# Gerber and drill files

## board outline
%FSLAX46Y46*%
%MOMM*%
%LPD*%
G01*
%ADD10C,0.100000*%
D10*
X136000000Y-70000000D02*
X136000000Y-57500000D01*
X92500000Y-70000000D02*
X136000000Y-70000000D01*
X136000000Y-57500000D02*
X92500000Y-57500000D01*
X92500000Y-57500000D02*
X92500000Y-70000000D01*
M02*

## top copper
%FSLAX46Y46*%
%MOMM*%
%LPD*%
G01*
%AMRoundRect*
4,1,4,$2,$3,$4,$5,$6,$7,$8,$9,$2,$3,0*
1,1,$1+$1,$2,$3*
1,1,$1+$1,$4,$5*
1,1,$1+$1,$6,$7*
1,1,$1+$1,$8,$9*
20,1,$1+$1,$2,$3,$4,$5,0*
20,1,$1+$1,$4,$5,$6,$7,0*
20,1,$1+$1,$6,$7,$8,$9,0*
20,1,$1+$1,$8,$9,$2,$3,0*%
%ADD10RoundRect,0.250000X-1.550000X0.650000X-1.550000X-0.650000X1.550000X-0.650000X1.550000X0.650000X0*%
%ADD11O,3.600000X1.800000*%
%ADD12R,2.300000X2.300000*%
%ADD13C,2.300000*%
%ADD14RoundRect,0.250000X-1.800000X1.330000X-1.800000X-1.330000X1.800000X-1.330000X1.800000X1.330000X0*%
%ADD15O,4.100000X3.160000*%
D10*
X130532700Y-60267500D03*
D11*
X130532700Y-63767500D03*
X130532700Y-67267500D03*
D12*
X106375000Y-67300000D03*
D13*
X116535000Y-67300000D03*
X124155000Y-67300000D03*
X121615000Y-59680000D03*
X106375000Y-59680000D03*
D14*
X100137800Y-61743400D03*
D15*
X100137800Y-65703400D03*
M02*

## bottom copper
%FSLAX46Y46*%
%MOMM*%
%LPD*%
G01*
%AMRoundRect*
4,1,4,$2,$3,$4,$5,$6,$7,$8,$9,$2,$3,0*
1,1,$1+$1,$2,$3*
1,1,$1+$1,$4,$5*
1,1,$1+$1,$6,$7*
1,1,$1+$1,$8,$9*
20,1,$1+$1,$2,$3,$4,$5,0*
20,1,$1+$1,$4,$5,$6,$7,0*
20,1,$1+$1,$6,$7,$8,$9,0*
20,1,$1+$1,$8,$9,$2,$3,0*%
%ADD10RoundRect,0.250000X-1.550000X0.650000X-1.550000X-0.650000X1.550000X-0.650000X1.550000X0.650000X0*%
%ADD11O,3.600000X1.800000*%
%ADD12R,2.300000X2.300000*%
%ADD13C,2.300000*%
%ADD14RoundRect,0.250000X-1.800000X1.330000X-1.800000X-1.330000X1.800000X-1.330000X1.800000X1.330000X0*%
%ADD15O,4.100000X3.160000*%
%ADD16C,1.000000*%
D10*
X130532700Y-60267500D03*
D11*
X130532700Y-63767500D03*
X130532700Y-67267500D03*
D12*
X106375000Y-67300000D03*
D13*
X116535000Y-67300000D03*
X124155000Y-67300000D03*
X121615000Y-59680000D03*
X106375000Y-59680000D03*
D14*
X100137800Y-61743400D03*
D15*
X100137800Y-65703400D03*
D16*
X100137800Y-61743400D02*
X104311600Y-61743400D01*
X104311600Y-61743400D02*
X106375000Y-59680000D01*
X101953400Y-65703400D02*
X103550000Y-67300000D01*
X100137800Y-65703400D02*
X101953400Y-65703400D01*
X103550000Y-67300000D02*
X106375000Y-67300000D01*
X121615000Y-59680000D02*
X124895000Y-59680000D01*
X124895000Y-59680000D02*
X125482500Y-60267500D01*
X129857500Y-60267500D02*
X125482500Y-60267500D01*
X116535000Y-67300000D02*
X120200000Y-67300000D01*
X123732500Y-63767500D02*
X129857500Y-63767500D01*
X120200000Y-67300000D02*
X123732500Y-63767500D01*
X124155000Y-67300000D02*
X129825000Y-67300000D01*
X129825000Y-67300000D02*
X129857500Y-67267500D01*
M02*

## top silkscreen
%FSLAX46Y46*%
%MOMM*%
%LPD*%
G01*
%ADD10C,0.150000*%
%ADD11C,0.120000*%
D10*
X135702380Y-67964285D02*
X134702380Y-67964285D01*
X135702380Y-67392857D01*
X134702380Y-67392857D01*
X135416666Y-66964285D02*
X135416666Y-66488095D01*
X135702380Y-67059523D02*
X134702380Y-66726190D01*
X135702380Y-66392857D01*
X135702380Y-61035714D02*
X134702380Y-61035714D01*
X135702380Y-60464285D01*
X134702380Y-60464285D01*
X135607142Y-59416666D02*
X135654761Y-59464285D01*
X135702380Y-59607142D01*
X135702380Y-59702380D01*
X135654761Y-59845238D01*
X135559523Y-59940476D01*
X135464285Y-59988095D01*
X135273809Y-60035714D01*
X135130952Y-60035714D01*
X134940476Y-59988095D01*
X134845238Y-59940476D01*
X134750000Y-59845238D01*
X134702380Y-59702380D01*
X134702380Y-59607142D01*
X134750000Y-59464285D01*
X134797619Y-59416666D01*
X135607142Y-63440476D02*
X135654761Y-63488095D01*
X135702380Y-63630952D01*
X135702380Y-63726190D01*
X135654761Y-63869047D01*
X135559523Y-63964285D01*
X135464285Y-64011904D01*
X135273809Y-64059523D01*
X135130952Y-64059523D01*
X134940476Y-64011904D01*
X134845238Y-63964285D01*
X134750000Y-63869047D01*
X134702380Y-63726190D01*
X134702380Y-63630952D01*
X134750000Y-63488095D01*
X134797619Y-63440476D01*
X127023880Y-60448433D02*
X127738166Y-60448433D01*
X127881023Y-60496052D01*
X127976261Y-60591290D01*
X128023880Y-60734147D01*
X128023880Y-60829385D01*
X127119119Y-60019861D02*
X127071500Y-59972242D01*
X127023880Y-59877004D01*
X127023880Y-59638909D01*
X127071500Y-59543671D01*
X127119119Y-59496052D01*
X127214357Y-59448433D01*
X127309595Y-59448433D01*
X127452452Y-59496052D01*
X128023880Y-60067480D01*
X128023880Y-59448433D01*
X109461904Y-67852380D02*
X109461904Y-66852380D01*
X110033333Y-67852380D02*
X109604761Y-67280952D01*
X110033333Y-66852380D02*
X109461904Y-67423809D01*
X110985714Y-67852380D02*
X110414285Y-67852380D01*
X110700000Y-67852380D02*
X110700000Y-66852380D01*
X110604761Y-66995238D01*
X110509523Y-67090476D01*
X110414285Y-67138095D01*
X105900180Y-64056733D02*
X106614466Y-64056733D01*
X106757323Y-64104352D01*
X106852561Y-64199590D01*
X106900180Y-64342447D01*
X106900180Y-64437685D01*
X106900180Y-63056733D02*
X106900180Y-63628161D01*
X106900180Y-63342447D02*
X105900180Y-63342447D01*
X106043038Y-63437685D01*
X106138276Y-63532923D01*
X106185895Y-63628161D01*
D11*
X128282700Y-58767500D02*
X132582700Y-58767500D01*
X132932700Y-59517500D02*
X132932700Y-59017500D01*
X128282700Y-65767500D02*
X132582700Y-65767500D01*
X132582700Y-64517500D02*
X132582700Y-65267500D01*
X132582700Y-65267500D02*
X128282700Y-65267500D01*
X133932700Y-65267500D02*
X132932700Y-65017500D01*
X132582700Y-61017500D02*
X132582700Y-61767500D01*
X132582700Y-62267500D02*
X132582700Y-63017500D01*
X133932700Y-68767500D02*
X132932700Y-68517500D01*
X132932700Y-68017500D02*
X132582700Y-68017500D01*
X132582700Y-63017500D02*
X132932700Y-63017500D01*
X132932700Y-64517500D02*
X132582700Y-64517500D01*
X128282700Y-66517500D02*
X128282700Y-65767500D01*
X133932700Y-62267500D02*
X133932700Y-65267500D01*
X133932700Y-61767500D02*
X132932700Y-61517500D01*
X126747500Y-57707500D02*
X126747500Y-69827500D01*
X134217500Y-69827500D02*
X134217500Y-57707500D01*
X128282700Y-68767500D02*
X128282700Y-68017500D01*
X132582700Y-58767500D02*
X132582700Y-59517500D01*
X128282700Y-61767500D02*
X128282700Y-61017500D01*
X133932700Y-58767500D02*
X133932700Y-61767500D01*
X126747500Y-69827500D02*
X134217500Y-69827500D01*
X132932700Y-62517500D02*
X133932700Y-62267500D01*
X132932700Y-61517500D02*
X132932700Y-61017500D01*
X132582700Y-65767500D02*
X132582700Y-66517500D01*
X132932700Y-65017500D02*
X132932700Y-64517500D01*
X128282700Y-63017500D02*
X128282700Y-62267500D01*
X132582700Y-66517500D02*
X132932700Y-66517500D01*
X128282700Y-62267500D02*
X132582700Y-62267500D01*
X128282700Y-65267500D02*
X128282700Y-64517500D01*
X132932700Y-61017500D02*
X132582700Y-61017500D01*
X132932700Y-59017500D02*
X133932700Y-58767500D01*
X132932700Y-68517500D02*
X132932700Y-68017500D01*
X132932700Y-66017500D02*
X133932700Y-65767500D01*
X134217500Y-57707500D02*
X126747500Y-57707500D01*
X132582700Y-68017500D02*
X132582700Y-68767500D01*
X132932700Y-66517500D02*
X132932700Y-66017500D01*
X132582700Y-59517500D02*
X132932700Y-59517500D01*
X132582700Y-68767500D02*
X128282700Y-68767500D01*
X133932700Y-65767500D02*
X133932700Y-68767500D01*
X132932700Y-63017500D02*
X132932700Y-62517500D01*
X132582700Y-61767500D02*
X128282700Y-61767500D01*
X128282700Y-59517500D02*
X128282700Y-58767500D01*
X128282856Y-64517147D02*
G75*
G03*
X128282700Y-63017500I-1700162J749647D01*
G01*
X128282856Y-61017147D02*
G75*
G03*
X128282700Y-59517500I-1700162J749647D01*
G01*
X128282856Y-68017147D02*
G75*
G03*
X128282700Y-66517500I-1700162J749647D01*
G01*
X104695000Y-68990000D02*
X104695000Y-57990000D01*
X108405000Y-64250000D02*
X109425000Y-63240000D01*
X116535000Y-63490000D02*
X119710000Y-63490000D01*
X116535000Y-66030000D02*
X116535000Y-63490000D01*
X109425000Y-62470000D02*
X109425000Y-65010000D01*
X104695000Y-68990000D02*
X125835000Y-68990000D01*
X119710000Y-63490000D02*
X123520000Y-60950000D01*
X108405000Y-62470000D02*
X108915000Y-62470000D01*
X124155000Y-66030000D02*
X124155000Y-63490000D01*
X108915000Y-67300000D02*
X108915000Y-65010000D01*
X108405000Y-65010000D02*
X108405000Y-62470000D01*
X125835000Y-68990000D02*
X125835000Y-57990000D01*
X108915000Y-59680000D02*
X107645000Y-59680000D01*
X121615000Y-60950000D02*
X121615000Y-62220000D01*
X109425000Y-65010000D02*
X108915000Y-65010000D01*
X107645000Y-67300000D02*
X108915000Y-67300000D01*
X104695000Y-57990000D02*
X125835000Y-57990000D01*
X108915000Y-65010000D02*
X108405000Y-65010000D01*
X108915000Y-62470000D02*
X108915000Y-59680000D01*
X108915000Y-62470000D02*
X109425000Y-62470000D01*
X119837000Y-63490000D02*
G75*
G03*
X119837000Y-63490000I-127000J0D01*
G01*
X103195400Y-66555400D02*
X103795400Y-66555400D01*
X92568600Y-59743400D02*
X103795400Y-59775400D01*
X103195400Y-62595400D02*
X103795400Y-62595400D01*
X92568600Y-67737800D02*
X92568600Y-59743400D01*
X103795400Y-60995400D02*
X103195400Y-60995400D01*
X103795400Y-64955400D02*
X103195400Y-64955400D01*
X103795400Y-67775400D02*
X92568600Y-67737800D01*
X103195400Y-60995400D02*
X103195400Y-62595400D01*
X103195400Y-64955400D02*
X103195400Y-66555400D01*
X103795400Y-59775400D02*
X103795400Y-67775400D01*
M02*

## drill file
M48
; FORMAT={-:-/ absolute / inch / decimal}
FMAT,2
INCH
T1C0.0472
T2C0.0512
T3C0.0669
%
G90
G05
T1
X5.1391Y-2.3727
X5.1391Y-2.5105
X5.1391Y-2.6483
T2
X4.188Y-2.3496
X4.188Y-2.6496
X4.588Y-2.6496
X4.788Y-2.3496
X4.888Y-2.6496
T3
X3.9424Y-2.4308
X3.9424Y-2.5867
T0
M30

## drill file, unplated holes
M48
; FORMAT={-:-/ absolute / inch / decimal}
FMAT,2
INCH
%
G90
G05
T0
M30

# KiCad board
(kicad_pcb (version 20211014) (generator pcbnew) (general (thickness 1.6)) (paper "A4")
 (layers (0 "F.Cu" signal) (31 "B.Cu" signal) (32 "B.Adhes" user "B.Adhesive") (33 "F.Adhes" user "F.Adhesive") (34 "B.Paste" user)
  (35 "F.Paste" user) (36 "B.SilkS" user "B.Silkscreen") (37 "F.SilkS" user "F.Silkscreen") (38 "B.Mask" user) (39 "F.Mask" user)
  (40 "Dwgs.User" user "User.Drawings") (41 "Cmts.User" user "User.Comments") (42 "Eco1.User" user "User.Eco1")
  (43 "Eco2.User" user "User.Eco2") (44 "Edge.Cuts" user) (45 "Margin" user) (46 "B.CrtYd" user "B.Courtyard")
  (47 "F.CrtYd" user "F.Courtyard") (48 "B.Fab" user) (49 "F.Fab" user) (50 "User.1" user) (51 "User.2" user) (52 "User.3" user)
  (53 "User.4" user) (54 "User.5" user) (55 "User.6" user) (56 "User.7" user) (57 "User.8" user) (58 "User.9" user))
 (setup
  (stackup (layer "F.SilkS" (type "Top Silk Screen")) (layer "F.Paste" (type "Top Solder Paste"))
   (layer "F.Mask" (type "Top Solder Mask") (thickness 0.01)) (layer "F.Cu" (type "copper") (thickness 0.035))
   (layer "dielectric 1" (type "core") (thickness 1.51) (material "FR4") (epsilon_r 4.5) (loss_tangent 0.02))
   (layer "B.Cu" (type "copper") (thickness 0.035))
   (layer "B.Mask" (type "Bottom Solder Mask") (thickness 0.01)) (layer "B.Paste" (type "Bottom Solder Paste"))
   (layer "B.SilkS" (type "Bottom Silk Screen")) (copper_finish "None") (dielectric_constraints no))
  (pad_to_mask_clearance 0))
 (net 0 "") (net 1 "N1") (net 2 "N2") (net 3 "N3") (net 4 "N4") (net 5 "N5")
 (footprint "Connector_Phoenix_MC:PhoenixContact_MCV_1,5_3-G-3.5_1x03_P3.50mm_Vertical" (layer "F.Cu") (at 129.8575 60.2675 -90)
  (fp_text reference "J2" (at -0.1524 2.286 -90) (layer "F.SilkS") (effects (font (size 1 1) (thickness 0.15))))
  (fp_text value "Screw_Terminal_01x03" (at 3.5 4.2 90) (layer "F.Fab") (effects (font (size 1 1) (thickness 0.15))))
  (fp_line (start -1.5 1.5748) (end -1.5 -2.7252) (layer "F.SilkS") (width 0.12))
  (fp_line (start -0.75 -3.0752) (end -1.25 -3.0752) (layer "F.SilkS") (width 0.12))
  (fp_line (start 5.5 1.5748) (end 5.5 -2.7252) (layer "F.SilkS") (width 0.12))
  (fp_line (start 4.25 -2.7252) (end 5 -2.7252) (layer "F.SilkS") (width 0.12))
  (fp_line (start 5 -2.7252) (end 5 1.5748) (layer "F.SilkS") (width 0.12))
  (fp_line (start 5 -4.0752) (end 4.75 -3.0752) (layer "F.SilkS") (width 0.12))
  (fp_line (start 0.75 -2.7252) (end 1.5 -2.7252) (layer "F.SilkS") (width 0.12))
  (fp_line (start 2 -2.7252) (end 2.75 -2.7252) (layer "F.SilkS") (width 0.12))
  (fp_line (start 8.5 -4.0752) (end 8.25 -3.0752) (layer "F.SilkS") (width 0.12))
  (fp_line (start 7.75 -3.0752) (end 7.75 -2.7252) (layer "F.SilkS") (width 0.12))
  (fp_line (start 2.75 -2.7252) (end 2.75 -3.0752) (layer "F.SilkS") (width 0.12))
  (fp_line (start 4.25 -3.0752) (end 4.25 -2.7252) (layer "F.SilkS") (width 0.12))
  (fp_line (start 6.25 1.5748) (end 5.5 1.5748) (layer "F.SilkS") (width 0.12))
  (fp_line (start 2 -4.0752) (end 5 -4.0752) (layer "F.SilkS") (width 0.12))
  (fp_line (start 1.5 -4.0752) (end 1.25 -3.0752) (layer "F.SilkS") (width 0.12))
  (fp_line (start -2.56 3.11) (end 9.56 3.11) (layer "F.SilkS") (width 0.12))
  (fp_line (start 9.56 -4.36) (end -2.56 -4.36) (layer "F.SilkS") (width 0.12))
  (fp_line (start 8.5 1.5748) (end 7.75 1.5748) (layer "F.SilkS") (width 0.12))
  (fp_line (start -1.5 -2.7252) (end -0.75 -2.7252) (layer "F.SilkS") (width 0.12))
  (fp_line (start 1.5 1.5748) (end 0.75 1.5748) (layer "F.SilkS") (width 0.12))
  (fp_line (start -1.5 -4.0752) (end 1.5 -4.0752) (layer "F.SilkS") (width 0.12))
  (fp_line (start 9.56 3.11) (end 9.56 -4.36) (layer "F.SilkS") (width 0.12))
  (fp_line (start 2.25 -3.0752) (end 2 -4.0752) (layer "F.SilkS") (width 0.12))
  (fp_line (start 1.25 -3.0752) (end 0.75 -3.0752) (layer "F.SilkS") (width 0.12))
  (fp_line (start 5.5 -2.7252) (end 6.25 -2.7252) (layer "F.SilkS") (width 0.12))
  (fp_line (start 4.75 -3.0752) (end 4.25 -3.0752) (layer "F.SilkS") (width 0.12))
  (fp_line (start 2.75 1.5748) (end 2 1.5748) (layer "F.SilkS") (width 0.12))
  (fp_line (start 6.25 -2.7252) (end 6.25 -3.0752) (layer "F.SilkS") (width 0.12))
  (fp_line (start 2 1.5748) (end 2 -2.7252) (layer "F.SilkS") (width 0.12))
  (fp_line (start 5 1.5748) (end 4.25 1.5748) (layer "F.SilkS") (width 0.12))
  (fp_line (start 0.75 -3.0752) (end 0.75 -2.7252) (layer "F.SilkS") (width 0.12))
  (fp_line (start -1.25 -3.0752) (end -1.5 -4.0752) (layer "F.SilkS") (width 0.12))
  (fp_line (start 8.25 -3.0752) (end 7.75 -3.0752) (layer "F.SilkS") (width 0.12))
  (fp_line (start 5.75 -3.0752) (end 5.5 -4.0752) (layer "F.SilkS") (width 0.12))
  (fp_line (start -2.56 -4.36) (end -2.56 3.11) (layer "F.SilkS") (width 0.12))
  (fp_line (start 7.75 -2.7252) (end 8.5 -2.7252) (layer "F.SilkS") (width 0.12))
  (fp_line (start 6.25 -3.0752) (end 5.75 -3.0752) (layer "F.SilkS") (width 0.12))
  (fp_line (start -0.75 -2.7252) (end -0.75 -3.0752) (layer "F.SilkS") (width 0.12))
  (fp_line (start 8.5 -2.7252) (end 8.5 1.5748) (layer "F.SilkS") (width 0.12))
  (fp_line (start 5.5 -4.0752) (end 8.5 -4.0752) (layer "F.SilkS") (width 0.12))
  (fp_line (start 2.75 -3.0752) (end 2.25 -3.0752) (layer "F.SilkS") (width 0.12))
  (fp_line (start 1.5 -2.7252) (end 1.5 1.5748) (layer "F.SilkS") (width 0.12))
  (fp_line (start -0.75 1.5748) (end -1.5 1.5748) (layer "F.SilkS") (width 0.12))
  (fp_arc (start 2.75 1.5748) (mid 3.499807 1.41671) (end 4.249647 1.574644) (layer "F.SilkS") (width 0.12))
  (fp_arc (start -0.75 1.5748) (mid -0.000193 1.41671) (end 0.749647 1.574644) (layer "F.SilkS") (width 0.12))
  (fp_arc (start 6.25 1.5748) (mid 6.999807 1.41671) (end 7.749647 1.574644) (layer "F.SilkS") (width 0.12))
  (pad "1" thru_hole roundrect (at 0 -0.6752 270) (size 1.8 3.6) (drill 1.2) (layers *.Cu *.Mask) (roundrect_rratio 0.1388888889)
   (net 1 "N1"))
  (pad "2" thru_hole oval (at 3.5 -0.6752 270) (size 1.8 3.6) (drill 1.2) (layers *.Cu *.Mask) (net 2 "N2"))
  (pad "3" thru_hole oval (at 7 -0.6752 270) (size 1.8 3.6) (drill 1.2) (layers *.Cu *.Mask) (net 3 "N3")))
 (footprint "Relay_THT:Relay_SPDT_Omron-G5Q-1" (layer "F.Cu") (at 106.375 67.3)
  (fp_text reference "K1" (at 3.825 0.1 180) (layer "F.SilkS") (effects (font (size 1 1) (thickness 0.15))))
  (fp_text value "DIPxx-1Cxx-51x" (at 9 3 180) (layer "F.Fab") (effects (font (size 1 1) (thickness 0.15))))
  (fp_line (start -1.68 1.69) (end -1.68 -9.31) (layer "F.SilkS") (width 0.12))
  (fp_line (start 2.03 -3.05) (end 3.05 -4.06) (layer "F.SilkS") (width 0.12))
  (fp_line (start 10.16 -3.81) (end 13.335 -3.81) (layer "F.SilkS") (width 0.12))
  (fp_line (start 10.16 -1.27) (end 10.16 -3.81) (layer "F.SilkS") (width 0.12))
  (fp_line (start 3.05 -4.83) (end 3.05 -2.29) (layer "F.SilkS") (width 0.12))
  (fp_line (start -1.68 1.69) (end 19.46 1.69) (layer "F.SilkS") (width 0.12))
  (fp_line (start 13.335 -3.81) (end 17.145 -6.35) (layer "F.SilkS") (width 0.12))
  (fp_line (start 2.03 -4.83) (end 2.54 -4.83) (layer "F.SilkS") (width 0.12))
  (fp_line (start 17.78 -1.27) (end 17.78 -3.81) (layer "F.SilkS") (width 0.12))
  (fp_line (start 2.54 0) (end 2.54 -2.29) (layer "F.SilkS") (width 0.12))
  (fp_line (start 2.03 -2.29) (end 2.03 -4.83) (layer "F.SilkS") (width 0.12))
  (fp_line (start 19.46 1.69) (end 19.46 -9.31) (layer "F.SilkS") (width 0.12))
  (fp_line (start 2.54 -7.62) (end 1.27 -7.62) (layer "F.SilkS") (width 0.12))
  (fp_line (start 15.24 -6.35) (end 15.24 -5.08) (layer "F.SilkS") (width 0.12))
  (fp_line (start 3.05 -2.29) (end 2.54 -2.29) (layer "F.SilkS") (width 0.12))
  (fp_line (start 1.27 0) (end 2.54 0) (layer "F.SilkS") (width 0.12))
  (fp_line (start -1.68 -9.31) (end 19.46 -9.31) (layer "F.SilkS") (width 0.12))
  (fp_line (start 2.54 -2.29) (end 2.03 -2.29) (layer "F.SilkS") (width 0.12))
  (fp_line (start 2.54 -4.83) (end 2.54 -7.62) (layer "F.SilkS") (width 0.12))
  (fp_line (start 2.54 -4.83) (end 3.05 -4.83) (layer "F.SilkS") (width 0.12))
  (fp_circle (center 13.335 -3.81) (end 13.462 -3.81) (layer "F.SilkS") (width 0.12) (fill none))
  (pad "1" thru_hole rect (at 0 0 180) (size 2.3 2.3) (drill 1.3) (layers *.Cu *.Mask) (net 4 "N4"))
  (pad "2" thru_hole circle (at 10.16 0 180) (size 2.3 2.3) (drill 1.3) (layers *.Cu *.Mask) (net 2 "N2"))
  (pad "3" thru_hole circle (at 17.78 0 180) (size 2.3 2.3) (drill 1.3) (layers *.Cu *.Mask) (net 3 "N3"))
  (pad "4" thru_hole circle (at 15.24 -7.62 180) (size 2.3 2.3) (drill 1.3) (layers *.Cu *.Mask) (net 1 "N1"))
  (pad "5" thru_hole circle (at 0 -7.62 180) (size 2.3 2.3) (drill 1.3) (layers *.Cu *.Mask) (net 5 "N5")))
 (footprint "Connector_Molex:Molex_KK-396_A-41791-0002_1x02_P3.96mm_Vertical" (layer "F.Cu") (at 100.1378 61.7434 -90)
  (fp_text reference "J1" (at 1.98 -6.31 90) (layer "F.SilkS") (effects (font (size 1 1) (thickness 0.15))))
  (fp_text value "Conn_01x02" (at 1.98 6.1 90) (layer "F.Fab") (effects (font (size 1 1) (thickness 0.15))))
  (fp_line (start 4.812 -3.0576) (end 4.812 -3.6576) (layer "F.SilkS") (width 0.12))
  (fp_line (start -2 7.5692) (end -1.968 -3.6576) (layer "F.SilkS") (width 0.12))
  (fp_line (start 0.852 -3.0576) (end 0.852 -3.6576) (layer "F.SilkS") (width 0.12))
  (fp_line (start 5.9944 7.5692) (end -2 7.5692) (layer "F.SilkS") (width 0.12))
  (fp_line (start -0.748 -3.6576) (end -0.748 -3.0576) (layer "F.SilkS") (width 0.12))
  (fp_line (start 3.212 -3.6576) (end 3.212 -3.0576) (layer "F.SilkS") (width 0.12))
  (fp_line (start 6.032 -3.6576) (end 5.9944 7.5692) (layer "F.SilkS") (width 0.12))
  (fp_line (start -0.748 -3.0576) (end 0.852 -3.0576) (layer "F.SilkS") (width 0.12))
  (fp_line (start 3.212 -3.0576) (end 4.812 -3.0576) (layer "F.SilkS") (width 0.12))
  (fp_line (start -1.968 -3.6576) (end 6.032 -3.6576) (layer "F.SilkS") (width 0.12))
  (pad "1" thru_hole roundrect (at 0 0 270) (size 3.16 4.1) (drill 1.7) (layers *.Cu *.Mask) (roundrect_rratio 0.07911392405) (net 5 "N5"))
  (pad "2" thru_hole oval (at 3.96 0 270) (size 3.16 4.1) (drill 1.7) (layers *.Cu *.Mask) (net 4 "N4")))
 (gr_line (start 136 70) (end 136 57.5) (layer "Edge.Cuts") (width 0.1))
 (gr_line (start 92.5 70) (end 136 70) (layer "Edge.Cuts") (width 0.1))
 (gr_line (start 136 57.5) (end 92.5 57.5) (layer "Edge.Cuts") (width 0.1))
 (gr_line (start 92.5 57.5) (end 92.5 70) (layer "Edge.Cuts") (width 0.1))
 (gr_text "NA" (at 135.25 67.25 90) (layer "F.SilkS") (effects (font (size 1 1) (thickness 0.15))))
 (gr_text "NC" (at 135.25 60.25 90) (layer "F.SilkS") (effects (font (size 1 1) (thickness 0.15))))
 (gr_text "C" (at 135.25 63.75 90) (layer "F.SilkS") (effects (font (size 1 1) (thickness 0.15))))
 (segment (start 100.1378 61.7434) (end 104.3116 61.7434) (width 1) (layer "B.Cu") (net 5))
 (segment (start 104.3116 61.7434) (end 106.375 59.68) (width 1) (layer "B.Cu") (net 5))
 (segment (start 101.9534 65.7034) (end 103.55 67.3) (width 1) (layer "B.Cu") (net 4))
 (segment (start 100.1378 65.7034) (end 101.9534 65.7034) (width 1) (layer "B.Cu") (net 4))
 (segment (start 103.55 67.3) (end 106.375 67.3) (width 1) (layer "B.Cu") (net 4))
 (segment (start 121.615 59.68) (end 124.895 59.68) (width 1) (layer "B.Cu") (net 1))
 (segment (start 124.895 59.68) (end 125.4825 60.2675) (width 1) (layer "B.Cu") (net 1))
 (segment (start 129.8575 60.2675) (end 125.4825 60.2675) (width 1) (layer "B.Cu") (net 1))
 (segment (start 116.535 67.3) (end 120.2 67.3) (width 1) (layer "B.Cu") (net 2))
 (segment (start 123.7325 63.7675) (end 129.8575 63.7675) (width 1) (layer "B.Cu") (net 2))
 (segment (start 120.2 67.3) (end 123.7325 63.7675) (width 1) (layer "B.Cu") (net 2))
 (segment (start 124.155 67.3) (end 129.825 67.3) (width 1) (layer "B.Cu") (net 3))
 (segment (start 129.825 67.3) (end 129.8575 67.2675) (width 1) (layer "B.Cu") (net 3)))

